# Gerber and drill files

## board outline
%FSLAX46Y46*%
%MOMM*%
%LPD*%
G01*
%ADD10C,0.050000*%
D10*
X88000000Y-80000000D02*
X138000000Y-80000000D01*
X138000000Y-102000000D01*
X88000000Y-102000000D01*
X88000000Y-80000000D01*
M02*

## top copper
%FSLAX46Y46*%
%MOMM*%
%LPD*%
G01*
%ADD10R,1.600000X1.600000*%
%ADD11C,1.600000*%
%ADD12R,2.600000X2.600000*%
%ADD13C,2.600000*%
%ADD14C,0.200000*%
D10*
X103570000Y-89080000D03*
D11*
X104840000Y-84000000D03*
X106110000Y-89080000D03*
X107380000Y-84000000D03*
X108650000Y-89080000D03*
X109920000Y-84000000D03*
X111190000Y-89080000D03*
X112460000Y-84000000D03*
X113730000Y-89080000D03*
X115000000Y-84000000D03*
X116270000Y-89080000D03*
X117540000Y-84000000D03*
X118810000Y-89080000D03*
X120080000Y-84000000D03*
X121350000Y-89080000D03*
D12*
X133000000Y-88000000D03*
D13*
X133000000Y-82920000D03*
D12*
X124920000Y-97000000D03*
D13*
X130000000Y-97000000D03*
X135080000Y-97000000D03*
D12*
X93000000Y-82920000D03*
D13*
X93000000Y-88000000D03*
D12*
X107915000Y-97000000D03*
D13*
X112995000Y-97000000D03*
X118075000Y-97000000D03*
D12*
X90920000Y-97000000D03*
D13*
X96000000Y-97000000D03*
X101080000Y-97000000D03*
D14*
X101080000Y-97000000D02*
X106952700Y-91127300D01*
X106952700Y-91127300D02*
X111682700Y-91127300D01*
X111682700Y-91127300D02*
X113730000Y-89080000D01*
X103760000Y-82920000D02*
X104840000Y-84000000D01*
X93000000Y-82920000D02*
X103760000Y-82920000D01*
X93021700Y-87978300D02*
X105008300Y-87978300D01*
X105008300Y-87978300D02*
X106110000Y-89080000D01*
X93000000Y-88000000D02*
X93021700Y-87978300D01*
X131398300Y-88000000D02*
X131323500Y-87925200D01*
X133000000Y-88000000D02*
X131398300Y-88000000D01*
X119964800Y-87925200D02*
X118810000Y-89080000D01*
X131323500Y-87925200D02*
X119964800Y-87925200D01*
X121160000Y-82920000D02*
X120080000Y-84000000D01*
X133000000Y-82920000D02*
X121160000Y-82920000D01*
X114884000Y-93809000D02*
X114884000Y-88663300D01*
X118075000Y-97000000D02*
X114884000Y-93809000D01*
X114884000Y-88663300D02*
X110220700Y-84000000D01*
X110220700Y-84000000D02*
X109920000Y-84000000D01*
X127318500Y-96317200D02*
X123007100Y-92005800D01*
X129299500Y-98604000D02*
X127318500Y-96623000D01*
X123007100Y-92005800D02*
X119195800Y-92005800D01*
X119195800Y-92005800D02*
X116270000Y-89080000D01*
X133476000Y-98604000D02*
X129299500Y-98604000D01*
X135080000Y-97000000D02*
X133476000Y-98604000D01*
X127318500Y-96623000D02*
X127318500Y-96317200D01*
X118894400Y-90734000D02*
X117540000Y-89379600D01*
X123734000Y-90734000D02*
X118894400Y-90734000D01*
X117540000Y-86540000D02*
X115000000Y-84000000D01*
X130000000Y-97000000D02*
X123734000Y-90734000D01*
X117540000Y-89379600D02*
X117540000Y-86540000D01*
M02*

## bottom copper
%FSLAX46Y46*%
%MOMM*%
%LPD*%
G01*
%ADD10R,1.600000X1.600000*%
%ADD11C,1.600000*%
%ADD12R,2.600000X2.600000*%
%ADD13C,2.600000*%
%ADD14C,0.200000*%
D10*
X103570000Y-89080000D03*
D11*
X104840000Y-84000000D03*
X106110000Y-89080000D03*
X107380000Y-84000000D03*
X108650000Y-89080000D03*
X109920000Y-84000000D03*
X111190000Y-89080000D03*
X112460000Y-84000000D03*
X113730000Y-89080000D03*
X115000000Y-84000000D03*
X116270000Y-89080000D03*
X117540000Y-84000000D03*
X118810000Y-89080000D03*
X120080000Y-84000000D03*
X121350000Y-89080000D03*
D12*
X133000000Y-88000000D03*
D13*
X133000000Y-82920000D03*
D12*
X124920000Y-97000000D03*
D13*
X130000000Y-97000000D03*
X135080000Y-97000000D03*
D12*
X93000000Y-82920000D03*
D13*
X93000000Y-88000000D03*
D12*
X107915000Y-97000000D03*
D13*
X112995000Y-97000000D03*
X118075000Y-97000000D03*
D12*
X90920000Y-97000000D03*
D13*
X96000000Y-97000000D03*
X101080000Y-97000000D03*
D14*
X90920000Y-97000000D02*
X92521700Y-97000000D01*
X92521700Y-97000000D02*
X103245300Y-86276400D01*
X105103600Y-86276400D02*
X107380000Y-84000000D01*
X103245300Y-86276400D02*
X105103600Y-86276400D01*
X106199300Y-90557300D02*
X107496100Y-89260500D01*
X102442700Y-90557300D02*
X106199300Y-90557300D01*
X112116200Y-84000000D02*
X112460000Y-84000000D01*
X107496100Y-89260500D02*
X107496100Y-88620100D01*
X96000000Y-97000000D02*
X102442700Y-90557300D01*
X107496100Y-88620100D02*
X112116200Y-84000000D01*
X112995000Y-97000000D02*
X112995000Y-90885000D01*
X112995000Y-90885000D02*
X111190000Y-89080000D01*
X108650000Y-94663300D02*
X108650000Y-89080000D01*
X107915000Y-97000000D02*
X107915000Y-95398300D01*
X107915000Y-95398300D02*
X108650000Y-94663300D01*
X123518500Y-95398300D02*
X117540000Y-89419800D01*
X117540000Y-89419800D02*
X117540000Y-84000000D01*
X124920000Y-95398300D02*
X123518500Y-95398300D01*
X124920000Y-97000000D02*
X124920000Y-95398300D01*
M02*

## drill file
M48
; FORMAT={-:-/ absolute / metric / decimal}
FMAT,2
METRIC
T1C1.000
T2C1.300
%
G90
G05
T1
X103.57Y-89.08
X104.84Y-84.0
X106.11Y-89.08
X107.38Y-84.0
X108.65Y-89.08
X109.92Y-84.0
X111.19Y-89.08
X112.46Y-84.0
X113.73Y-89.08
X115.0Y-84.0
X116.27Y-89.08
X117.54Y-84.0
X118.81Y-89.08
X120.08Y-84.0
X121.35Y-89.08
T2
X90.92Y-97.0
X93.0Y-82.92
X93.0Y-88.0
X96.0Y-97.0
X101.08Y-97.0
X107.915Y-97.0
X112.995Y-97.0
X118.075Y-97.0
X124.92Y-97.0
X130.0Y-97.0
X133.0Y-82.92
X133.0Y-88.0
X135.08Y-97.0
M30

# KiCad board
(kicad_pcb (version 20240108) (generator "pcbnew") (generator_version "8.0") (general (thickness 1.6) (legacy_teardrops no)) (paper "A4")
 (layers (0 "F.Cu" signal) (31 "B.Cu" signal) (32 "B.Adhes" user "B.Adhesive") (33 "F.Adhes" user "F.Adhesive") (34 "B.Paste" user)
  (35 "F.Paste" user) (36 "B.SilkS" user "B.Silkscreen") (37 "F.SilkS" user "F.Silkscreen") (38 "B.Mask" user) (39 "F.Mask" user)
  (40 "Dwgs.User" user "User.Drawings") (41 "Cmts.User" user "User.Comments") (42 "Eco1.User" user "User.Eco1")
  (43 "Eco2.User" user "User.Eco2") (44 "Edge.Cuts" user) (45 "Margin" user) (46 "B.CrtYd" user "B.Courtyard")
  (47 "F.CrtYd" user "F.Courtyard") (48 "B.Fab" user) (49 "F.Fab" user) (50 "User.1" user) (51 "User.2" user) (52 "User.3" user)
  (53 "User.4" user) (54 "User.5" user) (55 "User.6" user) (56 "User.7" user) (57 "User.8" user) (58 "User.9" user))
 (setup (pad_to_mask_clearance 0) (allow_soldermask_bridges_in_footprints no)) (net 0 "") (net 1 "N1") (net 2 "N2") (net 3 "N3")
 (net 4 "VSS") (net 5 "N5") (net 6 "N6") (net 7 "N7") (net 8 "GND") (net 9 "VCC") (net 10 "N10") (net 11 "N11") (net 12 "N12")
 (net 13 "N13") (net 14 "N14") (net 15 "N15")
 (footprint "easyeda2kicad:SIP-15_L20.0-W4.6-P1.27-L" (layer "F.Cu") (at 112.46 86.54)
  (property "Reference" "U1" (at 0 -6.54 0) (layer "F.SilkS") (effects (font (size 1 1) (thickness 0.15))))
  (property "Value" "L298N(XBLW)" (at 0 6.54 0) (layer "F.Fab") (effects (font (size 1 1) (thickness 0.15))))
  (pad "1" thru_hole rect (at -8.89 2.54) (size 1.6 1.6) (drill 0.999998) (layers "*.Cu" "*.Mask") (remove_unused_layers no) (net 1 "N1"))
  (pad "2" thru_hole circle (at -7.62 -2.54) (size 1.6 1.6) (drill 0.999998) (layers "*.Cu" "*.Mask") (remove_unused_layers no) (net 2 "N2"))
  (pad "3" thru_hole circle (at -6.35 2.54) (size 1.6 1.6) (drill 0.999998) (layers "*.Cu" "*.Mask") (remove_unused_layers no) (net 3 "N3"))
  (pad "4" thru_hole circle (at -5.08 -2.54) (size 1.6 1.6) (drill 0.999998) (layers "*.Cu" "*.Mask") (remove_unused_layers no)
   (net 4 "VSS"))
  (pad "5" thru_hole circle (at -3.81 2.54) (size 1.6 1.6) (drill 0.999998) (layers "*.Cu" "*.Mask") (remove_unused_layers no) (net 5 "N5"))
  (pad "6" thru_hole circle (at -2.54 -2.54) (size 1.6 1.6) (drill 0.999998) (layers "*.Cu" "*.Mask") (remove_unused_layers no) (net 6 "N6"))
  (pad "7" thru_hole circle (at -1.27 2.54) (size 1.6 1.6) (drill 0.999998) (layers "*.Cu" "*.Mask") (remove_unused_layers no) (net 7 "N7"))
  (pad "8" thru_hole circle (at 0 -2.54) (size 1.6 1.6) (drill 0.999998) (layers "*.Cu" "*.Mask") (remove_unused_layers no) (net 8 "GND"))
  (pad "9" thru_hole circle (at 1.27 2.54) (size 1.6 1.6) (drill 0.999998) (layers "*.Cu" "*.Mask") (remove_unused_layers no) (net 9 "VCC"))
  (pad "10" thru_hole circle (at 2.54 -2.54) (size 1.6 1.6) (drill 0.999998) (layers "*.Cu" "*.Mask") (remove_unused_layers no)
   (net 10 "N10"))
  (pad "11" thru_hole circle (at 3.81 2.54) (size 1.6 1.6) (drill 0.999998) (layers "*.Cu" "*.Mask") (remove_unused_layers no)
   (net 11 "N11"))
  (pad "12" thru_hole circle (at 5.08 -2.54) (size 1.6 1.6) (drill 0.999998) (layers "*.Cu" "*.Mask") (remove_unused_layers no)
   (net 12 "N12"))
  (pad "13" thru_hole circle (at 6.35 2.54) (size 1.6 1.6) (drill 0.999998) (layers "*.Cu" "*.Mask") (remove_unused_layers no)
   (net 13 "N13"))
  (pad "14" thru_hole circle (at 7.62 -2.54) (size 1.6 1.6) (drill 0.999998) (layers "*.Cu" "*.Mask") (remove_unused_layers no)
   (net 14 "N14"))
  (pad "15" thru_hole circle (at 8.89 2.54) (size 1.6 1.6) (drill 0.999998) (layers "*.Cu" "*.Mask") (remove_unused_layers no)
   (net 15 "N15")))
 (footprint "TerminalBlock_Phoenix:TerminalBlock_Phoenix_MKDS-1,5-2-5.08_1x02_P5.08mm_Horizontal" (layer "F.Cu") (at 133 88 90)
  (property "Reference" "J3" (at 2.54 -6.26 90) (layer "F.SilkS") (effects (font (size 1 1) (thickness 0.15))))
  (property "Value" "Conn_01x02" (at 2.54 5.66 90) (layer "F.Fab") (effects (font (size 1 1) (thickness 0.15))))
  (pad "1" thru_hole rect (at 0 0 90) (size 2.6 2.6) (drill 1.3) (layers "*.Cu" "*.Mask") (remove_unused_layers no) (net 13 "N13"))
  (pad "2" thru_hole circle (at 5.08 0 90) (size 2.6 2.6) (drill 1.3) (layers "*.Cu" "*.Mask") (remove_unused_layers no) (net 14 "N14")))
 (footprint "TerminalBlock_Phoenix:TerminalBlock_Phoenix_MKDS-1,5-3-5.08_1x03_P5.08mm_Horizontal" (layer "F.Cu") (at 124.92 97)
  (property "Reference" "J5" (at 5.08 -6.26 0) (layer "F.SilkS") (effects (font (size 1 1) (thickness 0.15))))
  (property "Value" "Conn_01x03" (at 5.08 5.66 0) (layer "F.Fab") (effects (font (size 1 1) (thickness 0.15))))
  (pad "1" thru_hole rect (at 0 0) (size 2.6 2.6) (drill 1.3) (layers "*.Cu" "*.Mask") (remove_unused_layers no) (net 12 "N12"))
  (pad "2" thru_hole circle (at 5.08 0) (size 2.6 2.6) (drill 1.3) (layers "*.Cu" "*.Mask") (remove_unused_layers no) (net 10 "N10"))
  (pad "3" thru_hole circle (at 10.16 0) (size 2.6 2.6) (drill 1.3) (layers "*.Cu" "*.Mask") (remove_unused_layers no) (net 11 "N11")))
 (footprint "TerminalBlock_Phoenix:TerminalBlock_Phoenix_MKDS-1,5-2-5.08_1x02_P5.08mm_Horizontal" (layer "F.Cu") (at 93 82.92 -90)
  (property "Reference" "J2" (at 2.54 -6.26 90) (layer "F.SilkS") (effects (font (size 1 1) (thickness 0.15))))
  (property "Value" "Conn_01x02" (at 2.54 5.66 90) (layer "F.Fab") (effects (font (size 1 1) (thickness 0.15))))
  (pad "1" thru_hole rect (at 0 0 270) (size 2.6 2.6) (drill 1.3) (layers "*.Cu" "*.Mask") (remove_unused_layers no) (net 2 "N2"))
  (pad "2" thru_hole circle (at 5.08 0 270) (size 2.6 2.6) (drill 1.3) (layers "*.Cu" "*.Mask") (remove_unused_layers no) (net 3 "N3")))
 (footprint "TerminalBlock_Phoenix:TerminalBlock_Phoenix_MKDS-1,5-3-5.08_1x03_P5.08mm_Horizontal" (layer "F.Cu") (at 107.915 97)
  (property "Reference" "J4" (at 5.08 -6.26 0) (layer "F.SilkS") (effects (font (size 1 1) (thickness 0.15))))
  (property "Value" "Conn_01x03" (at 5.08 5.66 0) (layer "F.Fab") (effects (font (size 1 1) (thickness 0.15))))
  (pad "1" thru_hole rect (at 0 0) (size 2.6 2.6) (drill 1.3) (layers "*.Cu" "*.Mask") (remove_unused_layers no) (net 5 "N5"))
  (pad "2" thru_hole circle (at 5.08 0) (size 2.6 2.6) (drill 1.3) (layers "*.Cu" "*.Mask") (remove_unused_layers no) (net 7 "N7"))
  (pad "3" thru_hole circle (at 10.16 0) (size 2.6 2.6) (drill 1.3) (layers "*.Cu" "*.Mask") (remove_unused_layers no) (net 6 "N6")))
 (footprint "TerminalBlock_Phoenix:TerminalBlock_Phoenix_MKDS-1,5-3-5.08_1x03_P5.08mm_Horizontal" (layer "F.Cu") (at 90.92 97)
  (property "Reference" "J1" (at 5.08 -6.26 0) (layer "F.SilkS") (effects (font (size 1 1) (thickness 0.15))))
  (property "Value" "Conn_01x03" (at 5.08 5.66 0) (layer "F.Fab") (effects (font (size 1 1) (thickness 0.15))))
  (pad "1" thru_hole rect (at 0 0) (size 2.6 2.6) (drill 1.3) (layers "*.Cu" "*.Mask") (remove_unused_layers no) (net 4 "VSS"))
  (pad "2" thru_hole circle (at 5.08 0) (size 2.6 2.6) (drill 1.3) (layers "*.Cu" "*.Mask") (remove_unused_layers no) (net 8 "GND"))
  (pad "3" thru_hole circle (at 10.16 0) (size 2.6 2.6) (drill 1.3) (layers "*.Cu" "*.Mask") (remove_unused_layers no) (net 9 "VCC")))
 (gr_rect (start 88 80) (end 138 102) (stroke (width 0.05) (type default)) (fill none) (layer "Edge.Cuts"))
 (segment (start 90.92 97) (end 92.5217 97) (width 0.2) (layer "B.Cu") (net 4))
 (segment (start 92.5217 97) (end 103.2453 86.2764) (width 0.2) (layer "B.Cu") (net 4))
 (segment (start 105.1036 86.2764) (end 107.38 84) (width 0.2) (layer "B.Cu") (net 4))
 (segment (start 103.2453 86.2764) (end 105.1036 86.2764) (width 0.2) (layer "B.Cu") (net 4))
 (segment (start 106.1993 90.5573) (end 107.4961 89.2605) (width 0.2) (layer "B.Cu") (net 8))
 (segment (start 102.4427 90.5573) (end 106.1993 90.5573) (width 0.2) (layer "B.Cu") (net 8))
 (segment (start 112.1162 84) (end 112.46 84) (width 0.2) (layer "B.Cu") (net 8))
 (segment (start 107.4961 89.2605) (end 107.4961 88.6201) (width 0.2) (layer "B.Cu") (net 8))
 (segment (start 96 97) (end 102.4427 90.5573) (width 0.2) (layer "B.Cu") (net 8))
 (segment (start 107.4961 88.6201) (end 112.1162 84) (width 0.2) (layer "B.Cu") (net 8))
 (segment (start 101.08 97) (end 106.9527 91.1273) (width 0.2) (layer "F.Cu") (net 9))
 (segment (start 106.9527 91.1273) (end 111.6827 91.1273) (width 0.2) (layer "F.Cu") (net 9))
 (segment (start 111.6827 91.1273) (end 113.73 89.08) (width 0.2) (layer "F.Cu") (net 9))
 (segment (start 103.76 82.92) (end 104.84 84) (width 0.2) (layer "F.Cu") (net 2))
 (segment (start 93 82.92) (end 103.76 82.92) (width 0.2) (layer "F.Cu") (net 2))
 (segment (start 93.0217 87.9783) (end 105.0083 87.9783) (width 0.2) (layer "F.Cu") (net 3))
 (segment (start 105.0083 87.9783) (end 106.11 89.08) (width 0.2) (layer "F.Cu") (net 3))
 (segment (start 93 88) (end 93.0217 87.9783) (width 0.2) (layer "F.Cu") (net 3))
 (segment (start 131.3983 88) (end 131.3235 87.9252) (width 0.2) (layer "F.Cu") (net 13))
 (segment (start 133 88) (end 131.3983 88) (width 0.2) (layer "F.Cu") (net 13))
 (segment (start 119.9648 87.9252) (end 118.81 89.08) (width 0.2) (layer "F.Cu") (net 13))
 (segment (start 131.3235 87.9252) (end 119.9648 87.9252) (width 0.2) (layer "F.Cu") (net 13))
 (segment (start 121.16 82.92) (end 120.08 84) (width 0.2) (layer "F.Cu") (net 14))
 (segment (start 133 82.92) (end 121.16 82.92) (width 0.2) (layer "F.Cu") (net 14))
 (segment (start 114.884 93.809) (end 114.884 88.6633) (width 0.2) (layer "F.Cu") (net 6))
 (segment (start 118.075 97) (end 114.884 93.809) (width 0.2) (layer "F.Cu") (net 6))
 (segment (start 114.884 88.6633) (end 110.2207 84) (width 0.2) (layer "F.Cu") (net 6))
 (segment (start 110.2207 84) (end 109.92 84) (width 0.2) (layer "F.Cu") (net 6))
 (segment (start 112.995 97) (end 112.995 90.885) (width 0.2) (layer "B.Cu") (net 7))
 (segment (start 112.995 90.885) (end 111.19 89.08) (width 0.2) (layer "B.Cu") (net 7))
 (segment (start 108.65 94.6633) (end 108.65 89.08) (width 0.2) (layer "B.Cu") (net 5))
 (segment (start 107.915 97) (end 107.915 95.3983) (width 0.2) (layer "B.Cu") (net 5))
 (segment (start 107.915 95.3983) (end 108.65 94.6633) (width 0.2) (layer "B.Cu") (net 5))
 (segment (start 127.3185 96.3172) (end 123.0071 92.0058) (width 0.2) (layer "F.Cu") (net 11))
 (segment (start 129.2995 98.604) (end 127.3185 96.623) (width 0.2) (layer "F.Cu") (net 11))
 (segment (start 123.0071 92.0058) (end 119.1958 92.0058) (width 0.2) (layer "F.Cu") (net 11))
 (segment (start 119.1958 92.0058) (end 116.27 89.08) (width 0.2) (layer "F.Cu") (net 11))
 (segment (start 133.476 98.604) (end 129.2995 98.604) (width 0.2) (layer "F.Cu") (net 11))
 (segment (start 135.08 97) (end 133.476 98.604) (width 0.2) (layer "F.Cu") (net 11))
 (segment (start 127.3185 96.623) (end 127.3185 96.3172) (width 0.2) (layer "F.Cu") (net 11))
 (segment (start 118.8944 90.734) (end 117.54 89.3796) (width 0.2) (layer "F.Cu") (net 10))
 (segment (start 123.734 90.734) (end 118.8944 90.734) (width 0.2) (layer "F.Cu") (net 10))
 (segment (start 117.54 86.54) (end 115 84) (width 0.2) (layer "F.Cu") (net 10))
 (segment (start 130 97) (end 123.734 90.734) (width 0.2) (layer "F.Cu") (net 10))
 (segment (start 117.54 89.3796) (end 117.54 86.54) (width 0.2) (layer "F.Cu") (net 10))
 (segment (start 123.5185 95.3983) (end 117.54 89.4198) (width 0.2) (layer "B.Cu") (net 12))
 (segment (start 117.54 89.4198) (end 117.54 84) (width 0.2) (layer "B.Cu") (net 12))
 (segment (start 124.92 95.3983) (end 123.5185 95.3983) (width 0.2) (layer "B.Cu") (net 12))
 (segment (start 124.92 97) (end 124.92 95.3983) (width 0.2) (layer "B.Cu") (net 12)))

